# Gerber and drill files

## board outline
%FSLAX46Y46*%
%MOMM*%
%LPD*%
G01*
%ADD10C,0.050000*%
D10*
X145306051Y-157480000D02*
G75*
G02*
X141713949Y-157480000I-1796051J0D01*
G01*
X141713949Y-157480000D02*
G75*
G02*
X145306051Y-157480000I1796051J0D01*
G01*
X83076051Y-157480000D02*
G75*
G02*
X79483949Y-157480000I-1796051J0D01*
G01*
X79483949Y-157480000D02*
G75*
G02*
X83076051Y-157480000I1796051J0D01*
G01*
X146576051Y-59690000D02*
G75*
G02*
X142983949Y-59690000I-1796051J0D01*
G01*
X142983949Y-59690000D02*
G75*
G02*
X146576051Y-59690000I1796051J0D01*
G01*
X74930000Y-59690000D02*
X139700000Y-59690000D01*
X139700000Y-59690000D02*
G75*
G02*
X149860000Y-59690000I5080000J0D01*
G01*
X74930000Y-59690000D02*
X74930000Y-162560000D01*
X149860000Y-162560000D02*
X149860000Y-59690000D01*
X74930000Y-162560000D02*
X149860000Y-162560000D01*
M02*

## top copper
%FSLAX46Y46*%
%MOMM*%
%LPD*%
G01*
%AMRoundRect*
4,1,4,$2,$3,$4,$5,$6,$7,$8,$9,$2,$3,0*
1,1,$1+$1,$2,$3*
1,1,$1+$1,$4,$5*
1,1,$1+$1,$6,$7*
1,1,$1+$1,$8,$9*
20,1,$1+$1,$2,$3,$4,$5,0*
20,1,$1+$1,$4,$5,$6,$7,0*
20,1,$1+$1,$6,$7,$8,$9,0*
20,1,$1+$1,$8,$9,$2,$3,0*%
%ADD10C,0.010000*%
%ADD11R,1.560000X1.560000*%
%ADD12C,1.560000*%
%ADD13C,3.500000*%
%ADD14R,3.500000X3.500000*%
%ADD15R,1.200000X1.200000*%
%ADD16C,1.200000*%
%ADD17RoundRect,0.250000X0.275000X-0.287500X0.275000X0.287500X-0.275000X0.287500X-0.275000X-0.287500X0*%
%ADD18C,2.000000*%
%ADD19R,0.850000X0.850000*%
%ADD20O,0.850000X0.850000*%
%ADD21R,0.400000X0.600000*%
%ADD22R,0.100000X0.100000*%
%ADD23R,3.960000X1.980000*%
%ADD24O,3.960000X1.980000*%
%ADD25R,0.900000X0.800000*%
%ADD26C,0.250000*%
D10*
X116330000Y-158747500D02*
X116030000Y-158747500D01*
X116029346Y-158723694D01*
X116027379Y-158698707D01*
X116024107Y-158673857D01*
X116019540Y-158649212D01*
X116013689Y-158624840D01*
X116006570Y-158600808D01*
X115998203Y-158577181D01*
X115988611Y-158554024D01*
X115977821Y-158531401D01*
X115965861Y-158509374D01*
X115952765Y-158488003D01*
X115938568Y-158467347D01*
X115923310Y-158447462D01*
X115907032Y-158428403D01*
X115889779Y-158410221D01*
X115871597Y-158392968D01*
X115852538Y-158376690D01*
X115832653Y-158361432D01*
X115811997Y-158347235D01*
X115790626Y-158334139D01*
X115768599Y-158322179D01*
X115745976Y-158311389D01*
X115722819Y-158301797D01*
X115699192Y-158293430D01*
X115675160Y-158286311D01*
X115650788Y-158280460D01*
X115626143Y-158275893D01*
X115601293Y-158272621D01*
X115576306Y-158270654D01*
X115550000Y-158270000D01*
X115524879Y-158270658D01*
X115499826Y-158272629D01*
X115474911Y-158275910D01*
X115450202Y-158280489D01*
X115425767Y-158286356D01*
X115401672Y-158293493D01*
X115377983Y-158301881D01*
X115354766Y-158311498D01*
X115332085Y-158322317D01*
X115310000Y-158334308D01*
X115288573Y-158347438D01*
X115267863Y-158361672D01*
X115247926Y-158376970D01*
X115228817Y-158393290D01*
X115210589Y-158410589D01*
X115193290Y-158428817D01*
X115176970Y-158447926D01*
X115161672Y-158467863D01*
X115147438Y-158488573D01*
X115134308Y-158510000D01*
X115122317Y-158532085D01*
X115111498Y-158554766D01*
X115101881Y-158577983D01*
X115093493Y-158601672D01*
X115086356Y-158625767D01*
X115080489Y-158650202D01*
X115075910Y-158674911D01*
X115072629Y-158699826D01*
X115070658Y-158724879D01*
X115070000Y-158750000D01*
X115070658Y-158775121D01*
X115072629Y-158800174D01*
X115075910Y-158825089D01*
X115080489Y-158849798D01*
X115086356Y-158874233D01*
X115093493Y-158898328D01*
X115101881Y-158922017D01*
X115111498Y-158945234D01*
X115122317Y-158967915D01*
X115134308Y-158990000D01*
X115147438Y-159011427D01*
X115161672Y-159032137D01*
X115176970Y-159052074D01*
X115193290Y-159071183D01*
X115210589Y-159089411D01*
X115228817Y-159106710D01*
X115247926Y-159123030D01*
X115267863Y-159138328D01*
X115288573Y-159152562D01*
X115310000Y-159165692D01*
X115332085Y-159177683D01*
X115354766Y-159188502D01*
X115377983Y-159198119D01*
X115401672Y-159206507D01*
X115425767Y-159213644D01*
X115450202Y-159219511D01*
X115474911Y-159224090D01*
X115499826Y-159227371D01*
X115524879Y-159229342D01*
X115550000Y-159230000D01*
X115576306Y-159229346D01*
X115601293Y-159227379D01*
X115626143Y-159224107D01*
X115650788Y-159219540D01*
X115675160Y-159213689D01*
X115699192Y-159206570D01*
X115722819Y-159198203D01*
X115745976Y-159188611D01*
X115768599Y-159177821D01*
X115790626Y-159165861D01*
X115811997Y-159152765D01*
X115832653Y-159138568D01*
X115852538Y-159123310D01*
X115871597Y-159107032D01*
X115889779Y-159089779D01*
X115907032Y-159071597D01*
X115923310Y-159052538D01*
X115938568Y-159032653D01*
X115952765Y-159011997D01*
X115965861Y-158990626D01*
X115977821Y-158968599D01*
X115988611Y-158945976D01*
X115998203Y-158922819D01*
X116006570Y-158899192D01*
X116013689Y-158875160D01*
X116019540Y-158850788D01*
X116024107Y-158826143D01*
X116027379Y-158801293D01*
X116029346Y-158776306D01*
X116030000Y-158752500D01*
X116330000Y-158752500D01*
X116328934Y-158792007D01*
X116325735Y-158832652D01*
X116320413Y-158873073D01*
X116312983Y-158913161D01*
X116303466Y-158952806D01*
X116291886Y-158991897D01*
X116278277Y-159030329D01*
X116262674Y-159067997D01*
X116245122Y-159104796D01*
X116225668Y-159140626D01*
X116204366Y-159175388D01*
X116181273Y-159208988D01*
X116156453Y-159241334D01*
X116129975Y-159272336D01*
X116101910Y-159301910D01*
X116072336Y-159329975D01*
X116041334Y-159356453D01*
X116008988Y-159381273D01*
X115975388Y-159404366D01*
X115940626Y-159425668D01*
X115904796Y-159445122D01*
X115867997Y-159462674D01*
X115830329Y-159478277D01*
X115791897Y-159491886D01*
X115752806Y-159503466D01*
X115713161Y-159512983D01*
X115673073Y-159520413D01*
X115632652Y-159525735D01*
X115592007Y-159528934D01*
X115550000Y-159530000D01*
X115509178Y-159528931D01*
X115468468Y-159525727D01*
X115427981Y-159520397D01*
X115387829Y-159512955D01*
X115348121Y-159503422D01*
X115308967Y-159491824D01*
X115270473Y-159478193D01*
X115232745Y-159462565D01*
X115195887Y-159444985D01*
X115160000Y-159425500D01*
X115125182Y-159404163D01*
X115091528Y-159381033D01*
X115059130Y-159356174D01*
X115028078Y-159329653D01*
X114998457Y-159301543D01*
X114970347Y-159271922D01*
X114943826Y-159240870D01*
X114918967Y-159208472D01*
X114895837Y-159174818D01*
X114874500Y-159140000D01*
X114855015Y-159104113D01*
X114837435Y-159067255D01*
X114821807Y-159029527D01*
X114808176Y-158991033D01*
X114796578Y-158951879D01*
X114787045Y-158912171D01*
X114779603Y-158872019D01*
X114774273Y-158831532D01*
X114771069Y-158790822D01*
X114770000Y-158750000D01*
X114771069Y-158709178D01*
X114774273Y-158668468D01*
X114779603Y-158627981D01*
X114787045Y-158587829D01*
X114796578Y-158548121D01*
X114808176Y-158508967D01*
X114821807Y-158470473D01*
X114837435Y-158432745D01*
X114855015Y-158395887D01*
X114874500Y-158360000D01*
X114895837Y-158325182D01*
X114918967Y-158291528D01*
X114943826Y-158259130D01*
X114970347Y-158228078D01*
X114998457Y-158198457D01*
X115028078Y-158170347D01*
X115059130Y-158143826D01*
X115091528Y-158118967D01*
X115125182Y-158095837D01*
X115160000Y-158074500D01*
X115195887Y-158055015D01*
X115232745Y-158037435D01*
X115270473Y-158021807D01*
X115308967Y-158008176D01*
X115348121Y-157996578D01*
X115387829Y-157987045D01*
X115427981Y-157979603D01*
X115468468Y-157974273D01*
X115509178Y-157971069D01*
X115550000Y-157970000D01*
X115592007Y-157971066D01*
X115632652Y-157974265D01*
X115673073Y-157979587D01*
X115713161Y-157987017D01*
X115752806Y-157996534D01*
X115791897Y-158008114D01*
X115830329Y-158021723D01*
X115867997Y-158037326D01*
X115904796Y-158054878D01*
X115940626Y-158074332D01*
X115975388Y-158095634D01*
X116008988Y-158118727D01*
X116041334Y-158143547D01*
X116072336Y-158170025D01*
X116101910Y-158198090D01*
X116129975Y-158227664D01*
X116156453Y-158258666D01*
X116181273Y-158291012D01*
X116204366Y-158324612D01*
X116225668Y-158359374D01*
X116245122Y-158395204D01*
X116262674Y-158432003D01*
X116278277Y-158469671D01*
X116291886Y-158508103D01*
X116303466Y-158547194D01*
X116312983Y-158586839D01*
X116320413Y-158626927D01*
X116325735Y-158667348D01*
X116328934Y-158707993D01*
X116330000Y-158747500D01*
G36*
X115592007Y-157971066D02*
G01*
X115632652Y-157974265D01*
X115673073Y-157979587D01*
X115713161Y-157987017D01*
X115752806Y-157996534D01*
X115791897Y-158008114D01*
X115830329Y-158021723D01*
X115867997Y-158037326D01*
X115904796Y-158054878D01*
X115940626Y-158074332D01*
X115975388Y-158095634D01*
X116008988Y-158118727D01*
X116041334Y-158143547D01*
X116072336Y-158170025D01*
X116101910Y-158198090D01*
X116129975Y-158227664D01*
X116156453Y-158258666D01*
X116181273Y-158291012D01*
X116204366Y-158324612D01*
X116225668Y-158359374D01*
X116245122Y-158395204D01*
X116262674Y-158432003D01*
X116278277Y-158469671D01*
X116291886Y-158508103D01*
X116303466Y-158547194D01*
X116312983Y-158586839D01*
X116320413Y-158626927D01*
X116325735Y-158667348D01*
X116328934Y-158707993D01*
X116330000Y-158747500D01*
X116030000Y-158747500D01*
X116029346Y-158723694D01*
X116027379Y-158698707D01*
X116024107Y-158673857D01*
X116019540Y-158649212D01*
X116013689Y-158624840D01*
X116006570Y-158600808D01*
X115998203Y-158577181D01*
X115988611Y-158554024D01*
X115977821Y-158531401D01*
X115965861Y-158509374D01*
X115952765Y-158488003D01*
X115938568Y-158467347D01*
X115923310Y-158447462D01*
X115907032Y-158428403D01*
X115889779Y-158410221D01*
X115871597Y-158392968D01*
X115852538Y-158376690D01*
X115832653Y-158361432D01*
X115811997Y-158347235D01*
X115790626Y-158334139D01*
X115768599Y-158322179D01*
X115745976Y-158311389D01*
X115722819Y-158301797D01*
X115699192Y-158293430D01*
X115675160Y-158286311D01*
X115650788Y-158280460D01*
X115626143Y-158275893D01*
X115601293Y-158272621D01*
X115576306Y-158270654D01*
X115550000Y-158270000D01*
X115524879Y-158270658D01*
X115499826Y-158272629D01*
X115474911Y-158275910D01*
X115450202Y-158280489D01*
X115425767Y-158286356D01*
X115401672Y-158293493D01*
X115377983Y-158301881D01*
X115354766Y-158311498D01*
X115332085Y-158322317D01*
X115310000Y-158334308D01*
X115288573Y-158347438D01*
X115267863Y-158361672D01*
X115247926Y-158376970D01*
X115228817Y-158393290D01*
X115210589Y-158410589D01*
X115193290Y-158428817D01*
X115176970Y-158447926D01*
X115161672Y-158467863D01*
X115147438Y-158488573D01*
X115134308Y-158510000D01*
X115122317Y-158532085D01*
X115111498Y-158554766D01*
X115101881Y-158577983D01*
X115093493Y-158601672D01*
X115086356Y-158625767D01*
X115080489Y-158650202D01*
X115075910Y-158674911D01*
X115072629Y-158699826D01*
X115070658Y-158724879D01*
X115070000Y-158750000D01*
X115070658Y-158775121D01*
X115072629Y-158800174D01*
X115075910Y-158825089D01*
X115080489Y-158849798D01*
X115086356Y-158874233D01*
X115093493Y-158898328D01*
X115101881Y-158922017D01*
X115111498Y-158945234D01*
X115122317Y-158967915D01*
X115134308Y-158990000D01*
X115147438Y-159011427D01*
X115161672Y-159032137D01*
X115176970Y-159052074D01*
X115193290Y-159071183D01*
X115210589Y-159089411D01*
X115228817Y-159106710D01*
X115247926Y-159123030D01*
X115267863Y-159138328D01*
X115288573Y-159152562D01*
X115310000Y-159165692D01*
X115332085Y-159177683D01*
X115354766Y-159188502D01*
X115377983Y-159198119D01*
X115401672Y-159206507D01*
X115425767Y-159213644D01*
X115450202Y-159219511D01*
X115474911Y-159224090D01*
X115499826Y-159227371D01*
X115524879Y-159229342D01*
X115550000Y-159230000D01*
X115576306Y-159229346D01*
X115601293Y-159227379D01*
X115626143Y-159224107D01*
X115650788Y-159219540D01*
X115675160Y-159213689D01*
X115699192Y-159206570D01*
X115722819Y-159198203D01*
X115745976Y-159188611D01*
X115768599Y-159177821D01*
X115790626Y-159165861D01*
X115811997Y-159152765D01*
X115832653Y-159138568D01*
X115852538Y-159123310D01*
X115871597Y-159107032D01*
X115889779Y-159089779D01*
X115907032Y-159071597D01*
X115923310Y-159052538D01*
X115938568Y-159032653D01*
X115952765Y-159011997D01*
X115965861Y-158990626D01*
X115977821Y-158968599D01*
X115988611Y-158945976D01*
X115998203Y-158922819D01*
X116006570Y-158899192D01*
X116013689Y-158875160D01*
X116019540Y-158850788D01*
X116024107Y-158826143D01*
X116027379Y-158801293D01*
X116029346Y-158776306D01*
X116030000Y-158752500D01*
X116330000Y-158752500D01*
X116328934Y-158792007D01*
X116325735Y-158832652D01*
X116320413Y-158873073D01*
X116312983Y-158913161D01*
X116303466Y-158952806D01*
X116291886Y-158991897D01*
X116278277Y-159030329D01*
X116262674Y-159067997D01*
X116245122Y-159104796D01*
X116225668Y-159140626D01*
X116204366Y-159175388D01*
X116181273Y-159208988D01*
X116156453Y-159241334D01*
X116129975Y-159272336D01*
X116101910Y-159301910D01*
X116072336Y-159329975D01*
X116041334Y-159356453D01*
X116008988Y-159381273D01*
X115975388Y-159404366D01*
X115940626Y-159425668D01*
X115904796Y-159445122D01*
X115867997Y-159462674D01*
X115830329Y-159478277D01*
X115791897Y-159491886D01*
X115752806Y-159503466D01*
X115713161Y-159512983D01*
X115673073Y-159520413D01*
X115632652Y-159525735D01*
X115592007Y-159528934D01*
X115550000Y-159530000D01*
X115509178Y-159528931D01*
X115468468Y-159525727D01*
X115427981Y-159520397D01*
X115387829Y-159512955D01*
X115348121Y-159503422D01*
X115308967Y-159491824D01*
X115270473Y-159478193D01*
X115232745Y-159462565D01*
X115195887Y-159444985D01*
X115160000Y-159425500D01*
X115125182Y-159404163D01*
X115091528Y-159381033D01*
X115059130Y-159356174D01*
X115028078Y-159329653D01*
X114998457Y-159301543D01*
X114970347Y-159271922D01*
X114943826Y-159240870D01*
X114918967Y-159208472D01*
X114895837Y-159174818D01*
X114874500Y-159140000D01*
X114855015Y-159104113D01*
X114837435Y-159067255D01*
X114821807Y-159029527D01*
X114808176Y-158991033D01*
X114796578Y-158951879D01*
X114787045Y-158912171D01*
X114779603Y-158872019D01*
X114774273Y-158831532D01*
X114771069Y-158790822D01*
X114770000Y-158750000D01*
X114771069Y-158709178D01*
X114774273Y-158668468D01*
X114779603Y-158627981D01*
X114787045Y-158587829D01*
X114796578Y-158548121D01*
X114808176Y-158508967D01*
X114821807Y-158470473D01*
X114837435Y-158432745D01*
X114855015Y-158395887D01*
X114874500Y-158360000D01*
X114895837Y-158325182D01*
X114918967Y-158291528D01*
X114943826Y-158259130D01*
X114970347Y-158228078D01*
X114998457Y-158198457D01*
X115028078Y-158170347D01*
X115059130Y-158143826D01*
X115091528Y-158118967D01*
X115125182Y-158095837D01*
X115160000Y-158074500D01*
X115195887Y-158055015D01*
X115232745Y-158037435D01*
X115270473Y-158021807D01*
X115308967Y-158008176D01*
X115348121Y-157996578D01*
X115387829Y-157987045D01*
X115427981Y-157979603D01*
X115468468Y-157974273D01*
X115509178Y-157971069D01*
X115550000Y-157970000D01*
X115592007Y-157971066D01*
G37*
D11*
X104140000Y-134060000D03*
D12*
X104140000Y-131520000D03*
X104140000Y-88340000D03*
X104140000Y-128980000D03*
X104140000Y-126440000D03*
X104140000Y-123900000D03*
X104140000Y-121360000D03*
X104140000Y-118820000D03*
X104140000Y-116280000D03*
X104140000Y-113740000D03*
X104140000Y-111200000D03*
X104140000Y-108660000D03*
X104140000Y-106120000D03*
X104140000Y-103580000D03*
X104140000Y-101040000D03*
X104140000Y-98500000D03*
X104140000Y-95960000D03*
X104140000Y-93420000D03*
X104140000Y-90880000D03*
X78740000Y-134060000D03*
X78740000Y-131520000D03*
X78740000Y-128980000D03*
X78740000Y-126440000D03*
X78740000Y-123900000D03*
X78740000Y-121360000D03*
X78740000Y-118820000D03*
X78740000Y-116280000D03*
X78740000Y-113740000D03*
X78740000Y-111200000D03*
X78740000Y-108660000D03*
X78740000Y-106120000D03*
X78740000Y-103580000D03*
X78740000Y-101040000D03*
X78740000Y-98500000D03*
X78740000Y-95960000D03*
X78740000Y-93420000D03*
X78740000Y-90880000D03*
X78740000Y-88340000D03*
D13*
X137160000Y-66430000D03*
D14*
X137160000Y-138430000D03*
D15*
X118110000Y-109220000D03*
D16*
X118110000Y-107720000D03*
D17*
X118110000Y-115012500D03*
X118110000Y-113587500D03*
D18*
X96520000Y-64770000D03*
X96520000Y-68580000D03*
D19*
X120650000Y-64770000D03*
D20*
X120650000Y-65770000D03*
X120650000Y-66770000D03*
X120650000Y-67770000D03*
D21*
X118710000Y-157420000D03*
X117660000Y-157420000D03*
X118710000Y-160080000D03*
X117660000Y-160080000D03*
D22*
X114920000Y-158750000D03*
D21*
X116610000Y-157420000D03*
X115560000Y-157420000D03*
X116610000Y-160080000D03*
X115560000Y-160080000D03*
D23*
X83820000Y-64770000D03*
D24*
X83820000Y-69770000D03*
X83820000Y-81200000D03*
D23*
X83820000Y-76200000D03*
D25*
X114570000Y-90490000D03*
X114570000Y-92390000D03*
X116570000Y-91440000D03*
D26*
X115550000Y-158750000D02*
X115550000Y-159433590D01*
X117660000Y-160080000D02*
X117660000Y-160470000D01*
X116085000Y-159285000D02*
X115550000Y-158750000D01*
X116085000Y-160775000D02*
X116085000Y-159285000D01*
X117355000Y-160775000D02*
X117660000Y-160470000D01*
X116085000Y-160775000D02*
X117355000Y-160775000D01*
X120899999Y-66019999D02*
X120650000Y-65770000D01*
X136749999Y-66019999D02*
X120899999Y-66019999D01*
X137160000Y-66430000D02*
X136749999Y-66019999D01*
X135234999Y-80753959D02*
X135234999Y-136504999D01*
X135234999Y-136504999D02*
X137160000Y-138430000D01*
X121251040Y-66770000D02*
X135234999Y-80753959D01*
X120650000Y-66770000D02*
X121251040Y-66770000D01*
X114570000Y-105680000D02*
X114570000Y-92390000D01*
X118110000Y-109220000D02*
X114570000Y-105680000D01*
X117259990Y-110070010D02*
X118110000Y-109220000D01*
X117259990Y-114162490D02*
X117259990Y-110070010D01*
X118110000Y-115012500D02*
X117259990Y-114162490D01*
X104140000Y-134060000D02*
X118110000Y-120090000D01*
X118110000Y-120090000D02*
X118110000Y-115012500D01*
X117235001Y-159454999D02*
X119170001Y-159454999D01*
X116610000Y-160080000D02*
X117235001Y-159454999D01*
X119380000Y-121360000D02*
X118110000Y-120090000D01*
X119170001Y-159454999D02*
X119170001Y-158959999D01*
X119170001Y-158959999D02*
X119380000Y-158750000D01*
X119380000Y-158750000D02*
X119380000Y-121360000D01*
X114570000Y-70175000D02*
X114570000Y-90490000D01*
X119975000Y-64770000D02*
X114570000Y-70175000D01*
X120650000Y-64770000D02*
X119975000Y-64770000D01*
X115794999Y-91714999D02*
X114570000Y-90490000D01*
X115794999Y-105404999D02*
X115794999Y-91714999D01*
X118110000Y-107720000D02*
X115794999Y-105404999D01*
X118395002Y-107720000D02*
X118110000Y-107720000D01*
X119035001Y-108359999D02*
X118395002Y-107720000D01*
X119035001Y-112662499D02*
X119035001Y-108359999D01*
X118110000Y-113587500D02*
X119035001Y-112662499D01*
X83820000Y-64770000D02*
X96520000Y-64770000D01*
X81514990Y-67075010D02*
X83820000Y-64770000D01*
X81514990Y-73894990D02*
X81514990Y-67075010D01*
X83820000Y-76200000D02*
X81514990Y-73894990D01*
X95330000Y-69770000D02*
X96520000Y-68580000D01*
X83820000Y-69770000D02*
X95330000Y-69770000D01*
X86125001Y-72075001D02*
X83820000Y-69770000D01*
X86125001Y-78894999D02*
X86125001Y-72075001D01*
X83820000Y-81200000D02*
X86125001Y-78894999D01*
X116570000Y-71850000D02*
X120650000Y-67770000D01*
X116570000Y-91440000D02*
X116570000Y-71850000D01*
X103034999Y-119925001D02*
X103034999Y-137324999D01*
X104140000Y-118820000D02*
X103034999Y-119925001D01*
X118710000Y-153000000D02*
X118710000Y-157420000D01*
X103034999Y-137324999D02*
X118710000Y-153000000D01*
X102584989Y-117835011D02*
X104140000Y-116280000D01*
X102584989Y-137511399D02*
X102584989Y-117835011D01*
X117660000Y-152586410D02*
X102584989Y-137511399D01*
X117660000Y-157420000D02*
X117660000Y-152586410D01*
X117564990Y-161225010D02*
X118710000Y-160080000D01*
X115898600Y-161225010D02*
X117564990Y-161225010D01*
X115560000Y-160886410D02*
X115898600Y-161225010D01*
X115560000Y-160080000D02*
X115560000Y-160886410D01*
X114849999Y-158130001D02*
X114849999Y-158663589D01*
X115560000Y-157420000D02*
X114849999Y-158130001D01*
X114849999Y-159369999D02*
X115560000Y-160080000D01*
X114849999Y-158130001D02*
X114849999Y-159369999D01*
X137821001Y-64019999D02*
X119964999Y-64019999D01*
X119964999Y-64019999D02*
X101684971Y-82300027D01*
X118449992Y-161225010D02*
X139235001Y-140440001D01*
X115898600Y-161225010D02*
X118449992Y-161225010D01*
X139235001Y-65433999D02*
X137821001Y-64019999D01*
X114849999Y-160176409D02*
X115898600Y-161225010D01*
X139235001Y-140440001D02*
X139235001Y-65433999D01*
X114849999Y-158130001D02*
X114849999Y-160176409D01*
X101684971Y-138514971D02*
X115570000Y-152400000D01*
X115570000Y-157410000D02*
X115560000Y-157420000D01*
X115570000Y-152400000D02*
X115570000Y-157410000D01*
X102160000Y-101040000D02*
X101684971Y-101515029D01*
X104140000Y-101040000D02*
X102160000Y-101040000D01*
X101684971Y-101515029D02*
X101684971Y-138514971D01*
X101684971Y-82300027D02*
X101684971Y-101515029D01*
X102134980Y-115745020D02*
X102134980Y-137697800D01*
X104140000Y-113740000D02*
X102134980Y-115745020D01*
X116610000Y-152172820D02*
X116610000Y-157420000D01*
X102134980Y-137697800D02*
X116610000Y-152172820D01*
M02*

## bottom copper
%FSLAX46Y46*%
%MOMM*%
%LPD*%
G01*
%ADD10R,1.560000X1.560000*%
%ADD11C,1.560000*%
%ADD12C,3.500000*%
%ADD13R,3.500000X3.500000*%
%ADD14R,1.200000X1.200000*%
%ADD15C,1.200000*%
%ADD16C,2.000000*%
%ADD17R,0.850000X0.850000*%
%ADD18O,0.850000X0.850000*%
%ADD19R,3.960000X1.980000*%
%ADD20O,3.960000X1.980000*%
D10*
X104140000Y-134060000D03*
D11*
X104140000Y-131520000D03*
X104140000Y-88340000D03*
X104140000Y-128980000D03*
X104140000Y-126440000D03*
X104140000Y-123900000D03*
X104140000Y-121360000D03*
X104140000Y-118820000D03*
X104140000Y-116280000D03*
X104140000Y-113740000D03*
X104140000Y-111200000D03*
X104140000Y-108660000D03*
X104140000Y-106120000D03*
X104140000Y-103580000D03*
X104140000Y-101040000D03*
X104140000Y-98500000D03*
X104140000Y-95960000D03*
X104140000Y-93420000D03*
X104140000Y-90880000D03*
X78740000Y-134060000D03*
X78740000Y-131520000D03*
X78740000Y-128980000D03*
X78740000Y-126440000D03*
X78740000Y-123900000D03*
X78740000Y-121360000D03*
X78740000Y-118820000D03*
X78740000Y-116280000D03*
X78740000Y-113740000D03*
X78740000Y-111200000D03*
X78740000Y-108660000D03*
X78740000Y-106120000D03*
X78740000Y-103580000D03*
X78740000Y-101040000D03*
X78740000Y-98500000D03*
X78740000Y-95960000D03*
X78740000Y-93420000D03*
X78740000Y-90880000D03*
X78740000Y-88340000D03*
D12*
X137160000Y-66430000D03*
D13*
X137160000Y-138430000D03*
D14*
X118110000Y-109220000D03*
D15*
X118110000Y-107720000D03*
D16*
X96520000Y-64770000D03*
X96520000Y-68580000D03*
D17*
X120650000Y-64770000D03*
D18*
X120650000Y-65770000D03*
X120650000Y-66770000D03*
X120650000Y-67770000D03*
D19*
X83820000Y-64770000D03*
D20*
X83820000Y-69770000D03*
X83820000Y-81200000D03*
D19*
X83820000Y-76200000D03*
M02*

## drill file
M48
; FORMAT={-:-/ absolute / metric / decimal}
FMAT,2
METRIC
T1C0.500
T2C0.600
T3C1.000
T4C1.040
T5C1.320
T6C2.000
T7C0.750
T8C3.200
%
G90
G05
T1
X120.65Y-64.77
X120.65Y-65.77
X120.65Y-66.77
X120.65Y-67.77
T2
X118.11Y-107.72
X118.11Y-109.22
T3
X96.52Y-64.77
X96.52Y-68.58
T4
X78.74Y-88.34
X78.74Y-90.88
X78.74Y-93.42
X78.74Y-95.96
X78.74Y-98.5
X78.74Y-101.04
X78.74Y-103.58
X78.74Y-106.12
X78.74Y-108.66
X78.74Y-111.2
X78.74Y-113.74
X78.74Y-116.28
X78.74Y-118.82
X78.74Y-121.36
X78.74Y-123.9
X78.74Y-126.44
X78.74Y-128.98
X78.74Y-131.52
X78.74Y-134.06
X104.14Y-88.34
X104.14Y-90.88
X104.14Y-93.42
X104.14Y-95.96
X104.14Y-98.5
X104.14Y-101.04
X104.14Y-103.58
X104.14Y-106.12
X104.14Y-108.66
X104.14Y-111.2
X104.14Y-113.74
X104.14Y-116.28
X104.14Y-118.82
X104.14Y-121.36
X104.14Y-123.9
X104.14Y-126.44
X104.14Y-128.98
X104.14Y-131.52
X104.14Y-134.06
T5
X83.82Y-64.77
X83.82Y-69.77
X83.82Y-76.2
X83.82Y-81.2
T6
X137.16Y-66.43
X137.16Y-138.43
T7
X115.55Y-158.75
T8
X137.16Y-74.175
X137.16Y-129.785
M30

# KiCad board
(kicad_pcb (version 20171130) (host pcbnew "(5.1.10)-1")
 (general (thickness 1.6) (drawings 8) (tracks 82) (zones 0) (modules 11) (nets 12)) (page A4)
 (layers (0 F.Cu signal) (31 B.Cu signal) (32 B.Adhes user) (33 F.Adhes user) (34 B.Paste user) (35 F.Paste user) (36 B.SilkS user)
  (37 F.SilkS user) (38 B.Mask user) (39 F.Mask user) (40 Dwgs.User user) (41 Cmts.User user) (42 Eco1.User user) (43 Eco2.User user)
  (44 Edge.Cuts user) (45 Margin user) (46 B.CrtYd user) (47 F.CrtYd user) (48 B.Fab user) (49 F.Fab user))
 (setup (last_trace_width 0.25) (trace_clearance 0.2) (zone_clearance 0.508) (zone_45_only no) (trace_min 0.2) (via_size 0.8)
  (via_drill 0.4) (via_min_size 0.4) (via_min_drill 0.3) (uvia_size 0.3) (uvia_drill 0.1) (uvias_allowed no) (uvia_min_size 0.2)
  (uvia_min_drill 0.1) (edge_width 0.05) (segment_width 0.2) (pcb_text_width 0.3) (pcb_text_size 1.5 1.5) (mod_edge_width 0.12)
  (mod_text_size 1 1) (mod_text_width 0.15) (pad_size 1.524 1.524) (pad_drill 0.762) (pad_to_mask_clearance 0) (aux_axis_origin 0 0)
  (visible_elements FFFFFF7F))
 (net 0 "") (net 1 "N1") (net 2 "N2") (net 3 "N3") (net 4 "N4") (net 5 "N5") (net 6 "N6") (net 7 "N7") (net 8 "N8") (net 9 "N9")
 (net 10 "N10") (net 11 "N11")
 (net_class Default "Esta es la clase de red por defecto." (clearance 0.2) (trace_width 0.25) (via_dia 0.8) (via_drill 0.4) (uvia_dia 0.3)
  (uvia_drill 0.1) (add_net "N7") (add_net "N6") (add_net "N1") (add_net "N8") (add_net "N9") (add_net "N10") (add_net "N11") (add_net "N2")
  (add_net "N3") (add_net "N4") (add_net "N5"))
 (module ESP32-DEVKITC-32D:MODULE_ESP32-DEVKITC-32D (layer F.Cu) (at 91.44 114.3 180)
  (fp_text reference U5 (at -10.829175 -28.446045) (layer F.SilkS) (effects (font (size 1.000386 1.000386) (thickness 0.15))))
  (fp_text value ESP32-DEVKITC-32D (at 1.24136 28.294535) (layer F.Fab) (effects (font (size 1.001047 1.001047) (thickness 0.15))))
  (pad 1 thru_hole rect (at -12.7 -19.76 180) (size 1.56 1.56) (drill 1.04) (layers *.Cu *.Mask) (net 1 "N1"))
  (pad 2 thru_hole circle (at -12.7 -17.22 180) (size 1.56 1.56) (drill 1.04) (layers *.Cu *.Mask))
  (pad 19 thru_hole circle (at -12.7 25.96 180) (size 1.56 1.56) (drill 1.04) (layers *.Cu *.Mask))
  (pad 3 thru_hole circle (at -12.7 -14.68 180) (size 1.56 1.56) (drill 1.04) (layers *.Cu *.Mask))
  (pad 4 thru_hole circle (at -12.7 -12.14 180) (size 1.56 1.56) (drill 1.04) (layers *.Cu *.Mask))
  (pad 5 thru_hole circle (at -12.7 -9.6 180) (size 1.56 1.56) (drill 1.04) (layers *.Cu *.Mask))
  (pad 6 thru_hole circle (at -12.7 -7.06 180) (size 1.56 1.56) (drill 1.04) (layers *.Cu *.Mask))
  (pad 7 thru_hole circle (at -12.7 -4.52 180) (size 1.56 1.56) (drill 1.04) (layers *.Cu *.Mask) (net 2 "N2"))
  (pad 8 thru_hole circle (at -12.7 -1.98 180) (size 1.56 1.56) (drill 1.04) (layers *.Cu *.Mask) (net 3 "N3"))
  (pad 9 thru_hole circle (at -12.7 0.56 180) (size 1.56 1.56) (drill 1.04) (layers *.Cu *.Mask) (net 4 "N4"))
  (pad 10 thru_hole circle (at -12.7 3.1 180) (size 1.56 1.56) (drill 1.04) (layers *.Cu *.Mask))
  (pad 11 thru_hole circle (at -12.7 5.64 180) (size 1.56 1.56) (drill 1.04) (layers *.Cu *.Mask))
  (pad 12 thru_hole circle (at -12.7 8.18 180) (size 1.56 1.56) (drill 1.04) (layers *.Cu *.Mask))
  (pad 13 thru_hole circle (at -12.7 10.72 180) (size 1.56 1.56) (drill 1.04) (layers *.Cu *.Mask))
  (pad 14 thru_hole circle (at -12.7 13.26 180) (size 1.56 1.56) (drill 1.04) (layers *.Cu *.Mask) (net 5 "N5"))
  (pad 15 thru_hole circle (at -12.7 15.8 180) (size 1.56 1.56) (drill 1.04) (layers *.Cu *.Mask))
  (pad 16 thru_hole circle (at -12.7 18.34 180) (size 1.56 1.56) (drill 1.04) (layers *.Cu *.Mask))
  (pad 17 thru_hole circle (at -12.7 20.88 180) (size 1.56 1.56) (drill 1.04) (layers *.Cu *.Mask))
  (pad 18 thru_hole circle (at -12.7 23.42 180) (size 1.56 1.56) (drill 1.04) (layers *.Cu *.Mask))
  (pad 20 thru_hole circle (at 12.7 -19.76 180) (size 1.56 1.56) (drill 1.04) (layers *.Cu *.Mask))
  (pad 21 thru_hole circle (at 12.7 -17.22 180) (size 1.56 1.56) (drill 1.04) (layers *.Cu *.Mask))
  (pad 22 thru_hole circle (at 12.7 -14.68 180) (size 1.56 1.56) (drill 1.04) (layers *.Cu *.Mask))
  (pad 23 thru_hole circle (at 12.7 -12.14 180) (size 1.56 1.56) (drill 1.04) (layers *.Cu *.Mask))
  (pad 24 thru_hole circle (at 12.7 -9.6 180) (size 1.56 1.56) (drill 1.04) (layers *.Cu *.Mask))
  (pad 25 thru_hole circle (at 12.7 -7.06 180) (size 1.56 1.56) (drill 1.04) (layers *.Cu *.Mask))
  (pad 26 thru_hole circle (at 12.7 -4.52 180) (size 1.56 1.56) (drill 1.04) (layers *.Cu *.Mask))
  (pad 27 thru_hole circle (at 12.7 -1.98 180) (size 1.56 1.56) (drill 1.04) (layers *.Cu *.Mask))
  (pad 28 thru_hole circle (at 12.7 0.56 180) (size 1.56 1.56) (drill 1.04) (layers *.Cu *.Mask))
  (pad 29 thru_hole circle (at 12.7 3.1 180) (size 1.56 1.56) (drill 1.04) (layers *.Cu *.Mask))
  (pad 30 thru_hole circle (at 12.7 5.64 180) (size 1.56 1.56) (drill 1.04) (layers *.Cu *.Mask))
  (pad 31 thru_hole circle (at 12.7 8.18 180) (size 1.56 1.56) (drill 1.04) (layers *.Cu *.Mask))
  (pad 32 thru_hole circle (at 12.7 10.72 180) (size 1.56 1.56) (drill 1.04) (layers *.Cu *.Mask))
  (pad 33 thru_hole circle (at 12.7 13.26 180) (size 1.56 1.56) (drill 1.04) (layers *.Cu *.Mask))
  (pad 34 thru_hole circle (at 12.7 15.8 180) (size 1.56 1.56) (drill 1.04) (layers *.Cu *.Mask))
  (pad 35 thru_hole circle (at 12.7 18.34 180) (size 1.56 1.56) (drill 1.04) (layers *.Cu *.Mask))
  (pad 36 thru_hole circle (at 12.7 20.88 180) (size 1.56 1.56) (drill 1.04) (layers *.Cu *.Mask))
  (pad 37 thru_hole circle (at 12.7 23.42 180) (size 1.56 1.56) (drill 1.04) (layers *.Cu *.Mask))
  (pad 38 thru_hole circle (at 12.7 25.96 180) (size 1.56 1.56) (drill 1.04) (layers *.Cu *.Mask)))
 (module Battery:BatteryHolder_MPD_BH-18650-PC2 (layer F.Cu) (at 137.16 138.43 90)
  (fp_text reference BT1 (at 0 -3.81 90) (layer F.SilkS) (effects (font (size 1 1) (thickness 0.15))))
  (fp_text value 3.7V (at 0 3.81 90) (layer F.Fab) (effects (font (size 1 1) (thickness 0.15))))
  (pad 2 thru_hole circle (at 72 0 90) (size 3.5 3.5) (drill 2) (layers *.Cu *.Mask) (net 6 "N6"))
  (pad 1 thru_hole rect (at 0 0 90) (size 3.5 3.5) (drill 2) (layers *.Cu *.Mask) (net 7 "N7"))
  (pad "" np_thru_hole circle (at 8.645 0 90) (size 3.2 3.2) (drill 3.2) (layers *.Cu *.Mask))
  (pad "" np_thru_hole circle (at 64.255 0 90) (size 3.2 3.2) (drill 3.2) (layers *.Cu *.Mask)))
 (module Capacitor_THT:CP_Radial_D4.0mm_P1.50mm (layer F.Cu) (at 118.11 109.22 90)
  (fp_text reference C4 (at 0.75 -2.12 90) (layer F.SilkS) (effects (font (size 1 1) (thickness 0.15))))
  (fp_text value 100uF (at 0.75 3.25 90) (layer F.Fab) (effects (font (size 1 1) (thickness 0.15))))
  (pad 1 thru_hole rect (at 0 0 90) (size 1.2 1.2) (drill 0.6) (layers *.Cu *.Mask) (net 1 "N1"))
  (pad 2 thru_hole circle (at 1.5 0 90) (size 1.2 1.2) (drill 0.6) (layers *.Cu *.Mask) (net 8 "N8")))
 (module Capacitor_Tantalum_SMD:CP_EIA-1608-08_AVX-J (layer F.Cu) (at 118.11 114.3 90)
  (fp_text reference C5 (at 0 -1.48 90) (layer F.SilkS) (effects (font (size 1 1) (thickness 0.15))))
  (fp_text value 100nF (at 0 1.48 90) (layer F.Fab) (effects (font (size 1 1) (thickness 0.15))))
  (pad 1 smd roundrect (at -0.7125 0 90) (size 1.075 1.05) (layers F.Cu F.Paste F.Mask) (roundrect_rratio 0.238095) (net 1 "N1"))
  (pad 2 smd roundrect (at 0.7125 0 90) (size 1.075 1.05) (layers F.Cu F.Paste F.Mask) (roundrect_rratio 0.238095) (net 8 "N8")))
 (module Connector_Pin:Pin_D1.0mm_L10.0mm (layer F.Cu) (at 96.52 64.77)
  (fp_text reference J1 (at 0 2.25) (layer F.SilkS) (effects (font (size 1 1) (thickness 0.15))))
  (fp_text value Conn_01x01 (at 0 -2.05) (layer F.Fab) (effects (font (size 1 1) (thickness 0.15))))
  (pad 1 thru_hole circle (at 0 0) (size 2 2) (drill 1) (layers *.Cu *.Mask) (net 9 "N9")))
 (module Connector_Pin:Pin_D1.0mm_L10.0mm (layer F.Cu) (at 96.52 68.58)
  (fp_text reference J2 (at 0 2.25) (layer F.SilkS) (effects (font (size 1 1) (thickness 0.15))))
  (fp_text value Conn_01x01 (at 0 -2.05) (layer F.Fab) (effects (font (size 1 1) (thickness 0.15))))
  (pad 1 thru_hole circle (at 0 0) (size 2 2) (drill 1) (layers *.Cu *.Mask) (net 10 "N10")))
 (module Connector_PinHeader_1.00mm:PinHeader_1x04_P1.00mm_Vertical (layer F.Cu) (at 120.65 64.77)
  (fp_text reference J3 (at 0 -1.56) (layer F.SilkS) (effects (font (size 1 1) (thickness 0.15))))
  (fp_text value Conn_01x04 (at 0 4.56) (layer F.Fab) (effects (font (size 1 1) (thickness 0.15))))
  (pad 1 thru_hole rect (at 0 0) (size 0.85 0.85) (drill 0.5) (layers *.Cu *.Mask) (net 8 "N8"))
  (pad 2 thru_hole oval (at 0 1) (size 0.85 0.85) (drill 0.5) (layers *.Cu *.Mask) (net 6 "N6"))
  (pad 3 thru_hole oval (at 0 2) (size 0.85 0.85) (drill 0.5) (layers *.Cu *.Mask) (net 7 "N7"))
  (pad 4 thru_hole oval (at 0 3) (size 0.85 0.85) (drill 0.5) (layers *.Cu *.Mask) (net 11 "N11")))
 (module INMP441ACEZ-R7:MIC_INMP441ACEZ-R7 (layer F.Cu) (at 116.84 158.75)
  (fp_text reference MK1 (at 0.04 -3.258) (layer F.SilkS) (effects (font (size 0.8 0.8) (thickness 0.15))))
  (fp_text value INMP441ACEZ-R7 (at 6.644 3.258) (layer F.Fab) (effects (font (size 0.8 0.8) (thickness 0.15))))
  (fp_poly
   (pts (xy -0.51 -0.0025) (xy -0.81 -0.0025) (xy -0.810654 -0.026306) (xy -0.812621 -0.051293) (xy -0.815893 -0.076143)
    (xy -0.82046 -0.100788) (xy -0.826311 -0.12516) (xy -0.83343 -0.149192) (xy -0.841797 -0.172819) (xy -0.851389 -0.195976)
    (xy -0.862179 -0.218599) (xy -0.874139 -0.240626) (xy -0.887235 -0.261997) (xy -0.901432 -0.282653) (xy -0.91669 -0.302538)
    (xy -0.932968 -0.321597) (xy -0.950221 -0.339779) (xy -0.968403 -0.357032) (xy -0.987462 -0.37331) (xy -1.007347 -0.388568)
    (xy -1.028003 -0.402765) (xy -1.049374 -0.415861) (xy -1.071401 -0.427821) (xy -1.094024 -0.438611) (xy -1.117181 -0.448203)
    (xy -1.140808 -0.45657) (xy -1.16484 -0.463689) (xy -1.189212 -0.46954) (xy -1.213857 -0.474107) (xy -1.238707 -0.477379)
    (xy -1.263694 -0.479346) (xy -1.29 -0.48) (xy -1.315121 -0.479342) (xy -1.340174 -0.477371) (xy -1.365089 -0.47409)
    (xy -1.389798 -0.469511) (xy -1.414233 -0.463644) (xy -1.438328 -0.456507) (xy -1.462017 -0.448119) (xy -1.485234 -0.438502)
    (xy -1.507915 -0.427683) (xy -1.53 -0.415692) (xy -1.551427 -0.402562) (xy -1.572137 -0.388328) (xy -1.592074 -0.37303)
    (xy -1.611183 -0.35671) (xy -1.629411 -0.339411) (xy -1.64671 -0.321183) (xy -1.66303 -0.302074) (xy -1.678328 -0.282137)
    (xy -1.692562 -0.261427) (xy -1.705692 -0.24) (xy -1.717683 -0.217915) (xy -1.728502 -0.195234) (xy -1.738119 -0.172017)
    (xy -1.746507 -0.148328) (xy -1.753644 -0.124233) (xy -1.759511 -0.099798) (xy -1.76409 -0.075089) (xy -1.767371 -0.050174)
    (xy -1.769342 -0.025121) (xy -1.77 0) (xy -1.769342 0.025121) (xy -1.767371 0.050174) (xy -1.76409 0.075089) (xy -1.759511 0.099798)
    (xy -1.753644 0.124233) (xy -1.746507 0.148328) (xy -1.738119 0.172017) (xy -1.728502 0.195234) (xy -1.717683 0.217915)
    (xy -1.705692 0.24) (xy -1.692562 0.261427) (xy -1.678328 0.282137) (xy -1.66303 0.302074) (xy -1.64671 0.321183)
    (xy -1.629411 0.339411) (xy -1.611183 0.35671) (xy -1.592074 0.37303) (xy -1.572137 0.388328) (xy -1.551427 0.402562)
    (xy -1.53 0.415692) (xy -1.507915 0.427683) (xy -1.485234 0.438502) (xy -1.462017 0.448119) (xy -1.438328 0.456507)
    (xy -1.414233 0.463644) (xy -1.389798 0.469511) (xy -1.365089 0.47409) (xy -1.340174 0.477371) (xy -1.315121 0.479342) (xy -1.29 0.48)
    (xy -1.263694 0.479346) (xy -1.238707 0.477379) (xy -1.213857 0.474107) (xy -1.189212 0.46954) (xy -1.16484 0.463689)
    (xy -1.140808 0.45657) (xy -1.117181 0.448203) (xy -1.094024 0.438611) (xy -1.071401 0.427821) (xy -1.049374 0.415861)
    (xy -1.028003 0.402765) (xy -1.007347 0.388568) (xy -0.987462 0.37331) (xy -0.968403 0.357032) (xy -0.950221 0.339779)
    (xy -0.932968 0.321597) (xy -0.91669 0.302538) (xy -0.901432 0.282653) (xy -0.887235 0.261997) (xy -0.874139 0.240626)
    (xy -0.862179 0.218599) (xy -0.851389 0.195976) (xy -0.841797 0.172819) (xy -0.83343 0.149192) (xy -0.826311 0.12516)
    (xy -0.82046 0.100788) (xy -0.815893 0.076143) (xy -0.812621 0.051293) (xy -0.810654 0.026306) (xy -0.81 0.0025) (xy -0.51 0.0025)
    (xy -0.511066 0.042007) (xy -0.514265 0.082652) (xy -0.519587 0.123073) (xy -0.527017 0.163161) (xy -0.536534 0.202806)
    (xy -0.548114 0.241897) (xy -0.561723 0.280329) (xy -0.577326 0.317997) (xy -0.594878 0.354796) (xy -0.614332 0.390626)
    (xy -0.635634 0.425388) (xy -0.658727 0.458988) (xy -0.683547 0.491334) (xy -0.710025 0.522336) (xy -0.73809 0.55191)
    (xy -0.767664 0.579975) (xy -0.798666 0.606453) (xy -0.831012 0.631273) (xy -0.864612 0.654366) (xy -0.899374 0.675668)
    (xy -0.935204 0.695122) (xy -0.972003 0.712674) (xy -1.009671 0.728277) (xy -1.048103 0.741886) (xy -1.087194 0.753466)
    (xy -1.126839 0.762983) (xy -1.166927 0.770413) (xy -1.207348 0.775735) (xy -1.247993 0.778934) (xy -1.29 0.78) (xy -1.330822 0.778931)
    (xy -1.371532 0.775727) (xy -1.412019 0.770397) (xy -1.452171 0.762955) (xy -1.491879 0.753422) (xy -1.531033 0.741824)
    (xy -1.569527 0.728193) (xy -1.607255 0.712565) (xy -1.644113 0.694985) (xy -1.68 0.6755) (xy -1.714818 0.654163)
    (xy -1.748472 0.631033) (xy -1.78087 0.606174) (xy -1.811922 0.579653) (xy -1.841543 0.551543) (xy -1.869653 0.521922)
    (xy -1.896174 0.49087) (xy -1.921033 0.458472) (xy -1.944163 0.424818) (xy -1.9655 0.39) (xy -1.984985 0.354113) (xy -2.002565 0.317255)
    (xy -2.018193 0.279527) (xy -2.031824 0.241033) (xy -2.043422 0.201879) (xy -2.052955 0.162171) (xy -2.060397 0.122019)
    (xy -2.065727 0.081532) (xy -2.068931 0.040822) (xy -2.07 0) (xy -2.068931 -0.040822) (xy -2.065727 -0.081532) (xy -2.060397 -0.122019)
    (xy -2.052955 -0.162171) (xy -2.043422 -0.201879) (xy -2.031824 -0.241033) (xy -2.018193 -0.279527) (xy -2.002565 -0.317255)
    (xy -1.984985 -0.354113) (xy -1.9655 -0.39) (xy -1.944163 -0.424818) (xy -1.921033 -0.458472) (xy -1.896174 -0.49087)
    (xy -1.869653 -0.521922) (xy -1.841543 -0.551543) (xy -1.811922 -0.579653) (xy -1.78087 -0.606174) (xy -1.748472 -0.631033)
    (xy -1.714818 -0.654163) (xy -1.68 -0.6755) (xy -1.644113 -0.694985) (xy -1.607255 -0.712565) (xy -1.569527 -0.728193)
    (xy -1.531033 -0.741824) (xy -1.491879 -0.753422) (xy -1.452171 -0.762955) (xy -1.412019 -0.770397) (xy -1.371532 -0.775727)
    (xy -1.330822 -0.778931) (xy -1.29 -0.78) (xy -1.247993 -0.778934) (xy -1.207348 -0.775735) (xy -1.166927 -0.770413)
    (xy -1.126839 -0.762983) (xy -1.087194 -0.753466) (xy -1.048103 -0.741886) (xy -1.009671 -0.728277) (xy -0.972003 -0.712674)
    (xy -0.935204 -0.695122) (xy -0.899374 -0.675668) (xy -0.864612 -0.654366) (xy -0.831012 -0.631273) (xy -0.798666 -0.606453)
    (xy -0.767664 -0.579975) (xy -0.73809 -0.55191) (xy -0.710025 -0.522336) (xy -0.683547 -0.491334) (xy -0.658727 -0.458988)
    (xy -0.635634 -0.425388) (xy -0.614332 -0.390626) (xy -0.594878 -0.354796) (xy -0.577326 -0.317997) (xy -0.561723 -0.280329)
    (xy -0.548114 -0.241897) (xy -0.536534 -0.202806) (xy -0.527017 -0.163161) (xy -0.519587 -0.123073) (xy -0.514265 -0.082652)
    (xy -0.511066 -0.042007) (xy -0.51 -0.0025))
   (layer F.Cu) (width 0.01))
  (pad 1 smd rect (at 1.87 -1.33) (size 0.4 0.6) (layers F.Cu F.Mask) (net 2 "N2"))
  (pad 2 smd rect (at 0.82 -1.33) (size 0.4 0.6) (layers F.Cu F.Mask) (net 3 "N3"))
  (pad 9 smd rect (at 1.87 1.33) (size 0.4 0.6) (layers F.Cu F.Mask) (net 5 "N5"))
  (pad 8 smd rect (at 0.82 1.33) (size 0.4 0.6) (layers F.Cu F.Mask))
  (pad 5 smd rect (at -1.92 0) (size 0.1 0.1) (layers F.Cu) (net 5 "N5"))
  (pad None np_thru_hole circle (at -1.29 0) (size 0.75 0.75) (drill 0.75) (layers *.Cu *.Mask))
  (pad 3 smd rect (at -0.23 -1.33) (size 0.4 0.6) (layers F.Cu F.Mask) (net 4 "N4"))
  (pad 4 smd rect (at -1.28 -1.33) (size 0.4 0.6) (layers F.Cu F.Mask) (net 5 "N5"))
  (pad 7 smd rect (at -0.23 1.33) (size 0.4 0.6) (layers F.Cu F.Mask) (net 1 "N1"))
  (pad 6 smd rect (at -1.28 1.33) (size 0.4 0.6) (layers F.Cu F.Mask) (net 5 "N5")))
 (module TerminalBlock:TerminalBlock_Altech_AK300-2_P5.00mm (layer F.Cu) (at 83.82 64.77 270)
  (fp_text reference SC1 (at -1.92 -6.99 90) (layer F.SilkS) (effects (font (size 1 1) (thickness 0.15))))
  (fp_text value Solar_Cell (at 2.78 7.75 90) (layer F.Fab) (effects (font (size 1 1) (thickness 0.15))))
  (pad 1 thru_hole rect (at 0 0 270) (size 1.98 3.96) (drill 1.32) (layers *.Cu *.Mask) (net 9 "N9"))
  (pad 2 thru_hole oval (at 5 0 270) (size 1.98 3.96) (drill 1.32) (layers *.Cu *.Mask) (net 10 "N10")))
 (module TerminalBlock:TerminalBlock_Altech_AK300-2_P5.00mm (layer F.Cu) (at 83.82 76.2 270)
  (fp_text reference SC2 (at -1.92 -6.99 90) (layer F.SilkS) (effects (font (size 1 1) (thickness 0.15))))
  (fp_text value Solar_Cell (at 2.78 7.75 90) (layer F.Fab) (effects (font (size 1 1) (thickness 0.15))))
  (pad 2 thru_hole oval (at 5 0 270) (size 1.98 3.96) (drill 1.32) (layers *.Cu *.Mask) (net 10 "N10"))
  (pad 1 thru_hole rect (at 0 0 270) (size 1.98 3.96) (drill 1.32) (layers *.Cu *.Mask) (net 9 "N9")))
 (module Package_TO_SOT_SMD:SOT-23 (layer F.Cu) (at 115.57 91.44)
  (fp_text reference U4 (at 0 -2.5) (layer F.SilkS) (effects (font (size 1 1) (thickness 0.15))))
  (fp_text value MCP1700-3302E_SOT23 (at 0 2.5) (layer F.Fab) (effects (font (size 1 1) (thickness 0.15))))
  (pad 1 smd rect (at -1 -0.95) (size 0.9 0.8) (layers F.Cu F.Paste F.Mask) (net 8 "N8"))
  (pad 2 smd rect (at -1 0.95) (size 0.9 0.8) (layers F.Cu F.Paste F.Mask) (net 1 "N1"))
  (pad 3 smd rect (at 1 0) (size 0.9 0.8) (layers F.Cu F.Paste F.Mask) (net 11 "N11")))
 (gr_circle (center 143.51 157.48) (end 144.78 156.21) (layer Edge.Cuts) (width 0.05))
 (gr_circle (center 81.28 157.48) (end 82.55 156.21) (layer Edge.Cuts) (width 0.05))
 (gr_circle (center 144.78 59.69) (end 146.05 58.42) (layer Edge.Cuts) (width 0.05))
 (gr_line (start 74.93 59.69) (end 139.7 59.69) (layer Edge.Cuts) (width 0.05))
 (gr_arc (start 144.78 59.69) (end 149.86 59.69) (angle -180) (layer Edge.Cuts) (width 0.05))
 (gr_line (start 74.93 59.69) (end 74.93 162.56) (layer Edge.Cuts) (width 0.05))
 (gr_line (start 149.86 162.56) (end 149.86 59.69) (layer Edge.Cuts) (width 0.05))
 (gr_line (start 74.93 162.56) (end 149.86 162.56) (layer Edge.Cuts) (width 0.05))
 (segment (start 115.55 158.75) (end 115.55 159.43359) (width 0.25) (layer F.Cu) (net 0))
 (segment (start 117.66 160.08) (end 117.66 160.47) (width 0.25) (layer F.Cu) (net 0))
 (segment (start 116.085 159.285) (end 115.55 158.75) (width 0.25) (layer F.Cu) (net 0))
 (segment (start 116.085 160.775) (end 116.085 159.285) (width 0.25) (layer F.Cu) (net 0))
 (segment (start 117.355 160.775) (end 117.66 160.47) (width 0.25) (layer F.Cu) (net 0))
 (segment (start 116.085 160.775) (end 117.355 160.775) (width 0.25) (layer F.Cu) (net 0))
 (segment (start 120.899999 66.019999) (end 120.65 65.77) (width 0.25) (layer F.Cu) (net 6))
 (segment (start 136.749999 66.019999) (end 120.899999 66.019999) (width 0.25) (layer F.Cu) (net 6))
 (segment (start 137.16 66.43) (end 136.749999 66.019999) (width 0.25) (layer F.Cu) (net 6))
 (segment (start 135.234999 80.753959) (end 135.234999 136.504999) (width 0.25) (layer F.Cu) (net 7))
 (segment (start 135.234999 136.504999) (end 137.16 138.43) (width 0.25) (layer F.Cu) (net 7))
 (segment (start 121.25104 66.77) (end 135.234999 80.753959) (width 0.25) (layer F.Cu) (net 7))
 (segment (start 120.65 66.77) (end 121.25104 66.77) (width 0.25) (layer F.Cu) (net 7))
 (segment (start 114.57 105.68) (end 114.57 92.39) (width 0.25) (layer F.Cu) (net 1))
 (segment (start 118.11 109.22) (end 114.57 105.68) (width 0.25) (layer F.Cu) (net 1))
 (segment (start 117.25999 110.07001) (end 118.11 109.22) (width 0.25) (layer F.Cu) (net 1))
 (segment (start 117.25999 114.16249) (end 117.25999 110.07001) (width 0.25) (layer F.Cu) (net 1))
 (segment (start 118.11 115.0125) (end 117.25999 114.16249) (width 0.25) (layer F.Cu) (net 1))
 (segment (start 104.14 134.06) (end 118.11 120.09) (width 0.25) (layer F.Cu) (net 1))
 (segment (start 118.11 120.09) (end 118.11 115.0125) (width 0.25) (layer F.Cu) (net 1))
 (segment (start 117.235001 159.454999) (end 119.170001 159.454999) (width 0.25) (layer F.Cu) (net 1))
 (segment (start 116.61 160.08) (end 117.235001 159.454999) (width 0.25) (layer F.Cu) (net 1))
 (segment (start 119.38 121.36) (end 118.11 120.09) (width 0.25) (layer F.Cu) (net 1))
 (segment (start 119.170001 159.454999) (end 119.170001 158.959999) (width 0.25) (layer F.Cu) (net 1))
 (segment (start 119.170001 158.959999) (end 119.38 158.75) (width 0.25) (layer F.Cu) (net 1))
 (segment (start 119.38 158.75) (end 119.38 121.36) (width 0.25) (layer F.Cu) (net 1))
 (segment (start 114.57 70.175) (end 114.57 90.49) (width 0.25) (layer F.Cu) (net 8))
 (segment (start 119.975 64.77) (end 114.57 70.175) (width 0.25) (layer F.Cu) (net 8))
 (segment (start 120.65 64.77) (end 119.975 64.77) (width 0.25) (layer F.Cu) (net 8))
 (segment (start 115.794999 91.714999) (end 114.57 90.49) (width 0.25) (layer F.Cu) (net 8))
 (segment (start 115.794999 105.404999) (end 115.794999 91.714999) (width 0.25) (layer F.Cu) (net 8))
 (segment (start 118.11 107.72) (end 115.794999 105.404999) (width 0.25) (layer F.Cu) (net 8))
 (segment (start 118.395002 107.72) (end 118.11 107.72) (width 0.25) (layer F.Cu) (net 8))
 (segment (start 119.035001 108.359999) (end 118.395002 107.72) (width 0.25) (layer F.Cu) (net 8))
 (segment (start 119.035001 112.662499) (end 119.035001 108.359999) (width 0.25) (layer F.Cu) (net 8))
 (segment (start 118.11 113.5875) (end 119.035001 112.662499) (width 0.25) (layer F.Cu) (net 8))
 (segment (start 83.82 64.77) (end 96.52 64.77) (width 0.25) (layer F.Cu) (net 9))
 (segment (start 81.51499 67.07501) (end 83.82 64.77) (width 0.25) (layer F.Cu) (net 9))
 (segment (start 81.51499 73.89499) (end 81.51499 67.07501) (width 0.25) (layer F.Cu) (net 9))
 (segment (start 83.82 76.2) (end 81.51499 73.89499) (width 0.25) (layer F.Cu) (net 9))
 (segment (start 95.33 69.77) (end 96.52 68.58) (width 0.25) (layer F.Cu) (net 10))
 (segment (start 83.82 69.77) (end 95.33 69.77) (width 0.25) (layer F.Cu) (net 10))
 (segment (start 86.125001 72.075001) (end 83.82 69.77) (width 0.25) (layer F.Cu) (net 10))
 (segment (start 86.125001 78.894999) (end 86.125001 72.075001) (width 0.25) (layer F.Cu) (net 10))
 (segment (start 83.82 81.2) (end 86.125001 78.894999) (width 0.25) (layer F.Cu) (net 10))
 (segment (start 116.57 71.85) (end 120.65 67.77) (width 0.25) (layer F.Cu) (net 11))
 (segment (start 116.57 91.44) (end 116.57 71.85) (width 0.25) (layer F.Cu) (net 11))
 (segment (start 103.034999 119.925001) (end 103.034999 137.324999) (width 0.25) (layer F.Cu) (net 2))
 (segment (start 104.14 118.82) (end 103.034999 119.925001) (width 0.25) (layer F.Cu) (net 2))
 (segment (start 118.71 153) (end 118.71 157.42) (width 0.25) (layer F.Cu) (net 2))
 (segment (start 103.034999 137.324999) (end 118.71 153) (width 0.25) (layer F.Cu) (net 2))
 (segment (start 102.584989 117.835011) (end 104.14 116.28) (width 0.25) (layer F.Cu) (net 3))
 (segment (start 102.584989 137.511399) (end 102.584989 117.835011) (width 0.25) (layer F.Cu) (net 3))
 (segment (start 117.66 152.58641) (end 102.584989 137.511399) (width 0.25) (layer F.Cu) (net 3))
 (segment (start 117.66 157.42) (end 117.66 152.58641) (width 0.25) (layer F.Cu) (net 3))
 (segment (start 117.56499 161.22501) (end 118.71 160.08) (width 0.25) (layer F.Cu) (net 5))
 (segment (start 115.8986 161.22501) (end 117.56499 161.22501) (width 0.25) (layer F.Cu) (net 5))
 (segment (start 115.56 160.88641) (end 115.8986 161.22501) (width 0.25) (layer F.Cu) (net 5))
 (segment (start 115.56 160.08) (end 115.56 160.88641) (width 0.25) (layer F.Cu) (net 5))
 (segment (start 114.849999 158.130001) (end 114.849999 158.663589) (width 0.25) (layer F.Cu) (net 5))
 (segment (start 115.56 157.42) (end 114.849999 158.130001) (width 0.25) (layer F.Cu) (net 5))
 (segment (start 114.849999 159.369999) (end 115.56 160.08) (width 0.25) (layer F.Cu) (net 5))
 (segment (start 114.849999 158.130001) (end 114.849999 159.369999) (width 0.25) (layer F.Cu) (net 5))
 (segment (start 137.821001 64.019999) (end 119.964999 64.019999) (width 0.25) (layer F.Cu) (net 5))
 (segment (start 119.964999 64.019999) (end 101.684971 82.300027) (width 0.25) (layer F.Cu) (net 5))
 (segment (start 118.449992 161.22501) (end 139.235001 140.440001) (width 0.25) (layer F.Cu) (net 5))
 (segment (start 115.8986 161.22501) (end 118.449992 161.22501) (width 0.25) (layer F.Cu) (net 5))
 (segment (start 139.235001 65.433999) (end 137.821001 64.019999) (width 0.25) (layer F.Cu) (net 5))
 (segment (start 114.849999 160.176409) (end 115.8986 161.22501) (width 0.25) (layer F.Cu) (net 5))
 (segment (start 139.235001 140.440001) (end 139.235001 65.433999) (width 0.25) (layer F.Cu) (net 5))
 (segment (start 114.849999 158.130001) (end 114.849999 160.176409) (width 0.25) (layer F.Cu) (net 5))
 (segment (start 101.684971 138.514971) (end 115.57 152.4) (width 0.25) (layer F.Cu) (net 5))
 (segment (start 115.57 157.41) (end 115.56 157.42) (width 0.25) (layer F.Cu) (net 5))
 (segment (start 115.57 152.4) (end 115.57 157.41) (width 0.25) (layer F.Cu) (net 5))
 (segment (start 102.16 101.04) (end 101.684971 101.515029) (width 0.25) (layer F.Cu) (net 5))
 (segment (start 104.14 101.04) (end 102.16 101.04) (width 0.25) (layer F.Cu) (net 5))
 (segment (start 101.684971 101.515029) (end 101.684971 138.514971) (width 0.25) (layer F.Cu) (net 5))
 (segment (start 101.684971 82.300027) (end 101.684971 101.515029) (width 0.25) (layer F.Cu) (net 5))
 (segment (start 102.13498 115.74502) (end 102.13498 137.6978) (width 0.25) (layer F.Cu) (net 4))
 (segment (start 104.14 113.74) (end 102.13498 115.74502) (width 0.25) (layer F.Cu) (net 4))
 (segment (start 116.61 152.17282) (end 116.61 157.42) (width 0.25) (layer F.Cu) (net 4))
 (segment (start 102.13498 137.6978) (end 116.61 152.17282) (width 0.25) (layer F.Cu) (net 4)))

